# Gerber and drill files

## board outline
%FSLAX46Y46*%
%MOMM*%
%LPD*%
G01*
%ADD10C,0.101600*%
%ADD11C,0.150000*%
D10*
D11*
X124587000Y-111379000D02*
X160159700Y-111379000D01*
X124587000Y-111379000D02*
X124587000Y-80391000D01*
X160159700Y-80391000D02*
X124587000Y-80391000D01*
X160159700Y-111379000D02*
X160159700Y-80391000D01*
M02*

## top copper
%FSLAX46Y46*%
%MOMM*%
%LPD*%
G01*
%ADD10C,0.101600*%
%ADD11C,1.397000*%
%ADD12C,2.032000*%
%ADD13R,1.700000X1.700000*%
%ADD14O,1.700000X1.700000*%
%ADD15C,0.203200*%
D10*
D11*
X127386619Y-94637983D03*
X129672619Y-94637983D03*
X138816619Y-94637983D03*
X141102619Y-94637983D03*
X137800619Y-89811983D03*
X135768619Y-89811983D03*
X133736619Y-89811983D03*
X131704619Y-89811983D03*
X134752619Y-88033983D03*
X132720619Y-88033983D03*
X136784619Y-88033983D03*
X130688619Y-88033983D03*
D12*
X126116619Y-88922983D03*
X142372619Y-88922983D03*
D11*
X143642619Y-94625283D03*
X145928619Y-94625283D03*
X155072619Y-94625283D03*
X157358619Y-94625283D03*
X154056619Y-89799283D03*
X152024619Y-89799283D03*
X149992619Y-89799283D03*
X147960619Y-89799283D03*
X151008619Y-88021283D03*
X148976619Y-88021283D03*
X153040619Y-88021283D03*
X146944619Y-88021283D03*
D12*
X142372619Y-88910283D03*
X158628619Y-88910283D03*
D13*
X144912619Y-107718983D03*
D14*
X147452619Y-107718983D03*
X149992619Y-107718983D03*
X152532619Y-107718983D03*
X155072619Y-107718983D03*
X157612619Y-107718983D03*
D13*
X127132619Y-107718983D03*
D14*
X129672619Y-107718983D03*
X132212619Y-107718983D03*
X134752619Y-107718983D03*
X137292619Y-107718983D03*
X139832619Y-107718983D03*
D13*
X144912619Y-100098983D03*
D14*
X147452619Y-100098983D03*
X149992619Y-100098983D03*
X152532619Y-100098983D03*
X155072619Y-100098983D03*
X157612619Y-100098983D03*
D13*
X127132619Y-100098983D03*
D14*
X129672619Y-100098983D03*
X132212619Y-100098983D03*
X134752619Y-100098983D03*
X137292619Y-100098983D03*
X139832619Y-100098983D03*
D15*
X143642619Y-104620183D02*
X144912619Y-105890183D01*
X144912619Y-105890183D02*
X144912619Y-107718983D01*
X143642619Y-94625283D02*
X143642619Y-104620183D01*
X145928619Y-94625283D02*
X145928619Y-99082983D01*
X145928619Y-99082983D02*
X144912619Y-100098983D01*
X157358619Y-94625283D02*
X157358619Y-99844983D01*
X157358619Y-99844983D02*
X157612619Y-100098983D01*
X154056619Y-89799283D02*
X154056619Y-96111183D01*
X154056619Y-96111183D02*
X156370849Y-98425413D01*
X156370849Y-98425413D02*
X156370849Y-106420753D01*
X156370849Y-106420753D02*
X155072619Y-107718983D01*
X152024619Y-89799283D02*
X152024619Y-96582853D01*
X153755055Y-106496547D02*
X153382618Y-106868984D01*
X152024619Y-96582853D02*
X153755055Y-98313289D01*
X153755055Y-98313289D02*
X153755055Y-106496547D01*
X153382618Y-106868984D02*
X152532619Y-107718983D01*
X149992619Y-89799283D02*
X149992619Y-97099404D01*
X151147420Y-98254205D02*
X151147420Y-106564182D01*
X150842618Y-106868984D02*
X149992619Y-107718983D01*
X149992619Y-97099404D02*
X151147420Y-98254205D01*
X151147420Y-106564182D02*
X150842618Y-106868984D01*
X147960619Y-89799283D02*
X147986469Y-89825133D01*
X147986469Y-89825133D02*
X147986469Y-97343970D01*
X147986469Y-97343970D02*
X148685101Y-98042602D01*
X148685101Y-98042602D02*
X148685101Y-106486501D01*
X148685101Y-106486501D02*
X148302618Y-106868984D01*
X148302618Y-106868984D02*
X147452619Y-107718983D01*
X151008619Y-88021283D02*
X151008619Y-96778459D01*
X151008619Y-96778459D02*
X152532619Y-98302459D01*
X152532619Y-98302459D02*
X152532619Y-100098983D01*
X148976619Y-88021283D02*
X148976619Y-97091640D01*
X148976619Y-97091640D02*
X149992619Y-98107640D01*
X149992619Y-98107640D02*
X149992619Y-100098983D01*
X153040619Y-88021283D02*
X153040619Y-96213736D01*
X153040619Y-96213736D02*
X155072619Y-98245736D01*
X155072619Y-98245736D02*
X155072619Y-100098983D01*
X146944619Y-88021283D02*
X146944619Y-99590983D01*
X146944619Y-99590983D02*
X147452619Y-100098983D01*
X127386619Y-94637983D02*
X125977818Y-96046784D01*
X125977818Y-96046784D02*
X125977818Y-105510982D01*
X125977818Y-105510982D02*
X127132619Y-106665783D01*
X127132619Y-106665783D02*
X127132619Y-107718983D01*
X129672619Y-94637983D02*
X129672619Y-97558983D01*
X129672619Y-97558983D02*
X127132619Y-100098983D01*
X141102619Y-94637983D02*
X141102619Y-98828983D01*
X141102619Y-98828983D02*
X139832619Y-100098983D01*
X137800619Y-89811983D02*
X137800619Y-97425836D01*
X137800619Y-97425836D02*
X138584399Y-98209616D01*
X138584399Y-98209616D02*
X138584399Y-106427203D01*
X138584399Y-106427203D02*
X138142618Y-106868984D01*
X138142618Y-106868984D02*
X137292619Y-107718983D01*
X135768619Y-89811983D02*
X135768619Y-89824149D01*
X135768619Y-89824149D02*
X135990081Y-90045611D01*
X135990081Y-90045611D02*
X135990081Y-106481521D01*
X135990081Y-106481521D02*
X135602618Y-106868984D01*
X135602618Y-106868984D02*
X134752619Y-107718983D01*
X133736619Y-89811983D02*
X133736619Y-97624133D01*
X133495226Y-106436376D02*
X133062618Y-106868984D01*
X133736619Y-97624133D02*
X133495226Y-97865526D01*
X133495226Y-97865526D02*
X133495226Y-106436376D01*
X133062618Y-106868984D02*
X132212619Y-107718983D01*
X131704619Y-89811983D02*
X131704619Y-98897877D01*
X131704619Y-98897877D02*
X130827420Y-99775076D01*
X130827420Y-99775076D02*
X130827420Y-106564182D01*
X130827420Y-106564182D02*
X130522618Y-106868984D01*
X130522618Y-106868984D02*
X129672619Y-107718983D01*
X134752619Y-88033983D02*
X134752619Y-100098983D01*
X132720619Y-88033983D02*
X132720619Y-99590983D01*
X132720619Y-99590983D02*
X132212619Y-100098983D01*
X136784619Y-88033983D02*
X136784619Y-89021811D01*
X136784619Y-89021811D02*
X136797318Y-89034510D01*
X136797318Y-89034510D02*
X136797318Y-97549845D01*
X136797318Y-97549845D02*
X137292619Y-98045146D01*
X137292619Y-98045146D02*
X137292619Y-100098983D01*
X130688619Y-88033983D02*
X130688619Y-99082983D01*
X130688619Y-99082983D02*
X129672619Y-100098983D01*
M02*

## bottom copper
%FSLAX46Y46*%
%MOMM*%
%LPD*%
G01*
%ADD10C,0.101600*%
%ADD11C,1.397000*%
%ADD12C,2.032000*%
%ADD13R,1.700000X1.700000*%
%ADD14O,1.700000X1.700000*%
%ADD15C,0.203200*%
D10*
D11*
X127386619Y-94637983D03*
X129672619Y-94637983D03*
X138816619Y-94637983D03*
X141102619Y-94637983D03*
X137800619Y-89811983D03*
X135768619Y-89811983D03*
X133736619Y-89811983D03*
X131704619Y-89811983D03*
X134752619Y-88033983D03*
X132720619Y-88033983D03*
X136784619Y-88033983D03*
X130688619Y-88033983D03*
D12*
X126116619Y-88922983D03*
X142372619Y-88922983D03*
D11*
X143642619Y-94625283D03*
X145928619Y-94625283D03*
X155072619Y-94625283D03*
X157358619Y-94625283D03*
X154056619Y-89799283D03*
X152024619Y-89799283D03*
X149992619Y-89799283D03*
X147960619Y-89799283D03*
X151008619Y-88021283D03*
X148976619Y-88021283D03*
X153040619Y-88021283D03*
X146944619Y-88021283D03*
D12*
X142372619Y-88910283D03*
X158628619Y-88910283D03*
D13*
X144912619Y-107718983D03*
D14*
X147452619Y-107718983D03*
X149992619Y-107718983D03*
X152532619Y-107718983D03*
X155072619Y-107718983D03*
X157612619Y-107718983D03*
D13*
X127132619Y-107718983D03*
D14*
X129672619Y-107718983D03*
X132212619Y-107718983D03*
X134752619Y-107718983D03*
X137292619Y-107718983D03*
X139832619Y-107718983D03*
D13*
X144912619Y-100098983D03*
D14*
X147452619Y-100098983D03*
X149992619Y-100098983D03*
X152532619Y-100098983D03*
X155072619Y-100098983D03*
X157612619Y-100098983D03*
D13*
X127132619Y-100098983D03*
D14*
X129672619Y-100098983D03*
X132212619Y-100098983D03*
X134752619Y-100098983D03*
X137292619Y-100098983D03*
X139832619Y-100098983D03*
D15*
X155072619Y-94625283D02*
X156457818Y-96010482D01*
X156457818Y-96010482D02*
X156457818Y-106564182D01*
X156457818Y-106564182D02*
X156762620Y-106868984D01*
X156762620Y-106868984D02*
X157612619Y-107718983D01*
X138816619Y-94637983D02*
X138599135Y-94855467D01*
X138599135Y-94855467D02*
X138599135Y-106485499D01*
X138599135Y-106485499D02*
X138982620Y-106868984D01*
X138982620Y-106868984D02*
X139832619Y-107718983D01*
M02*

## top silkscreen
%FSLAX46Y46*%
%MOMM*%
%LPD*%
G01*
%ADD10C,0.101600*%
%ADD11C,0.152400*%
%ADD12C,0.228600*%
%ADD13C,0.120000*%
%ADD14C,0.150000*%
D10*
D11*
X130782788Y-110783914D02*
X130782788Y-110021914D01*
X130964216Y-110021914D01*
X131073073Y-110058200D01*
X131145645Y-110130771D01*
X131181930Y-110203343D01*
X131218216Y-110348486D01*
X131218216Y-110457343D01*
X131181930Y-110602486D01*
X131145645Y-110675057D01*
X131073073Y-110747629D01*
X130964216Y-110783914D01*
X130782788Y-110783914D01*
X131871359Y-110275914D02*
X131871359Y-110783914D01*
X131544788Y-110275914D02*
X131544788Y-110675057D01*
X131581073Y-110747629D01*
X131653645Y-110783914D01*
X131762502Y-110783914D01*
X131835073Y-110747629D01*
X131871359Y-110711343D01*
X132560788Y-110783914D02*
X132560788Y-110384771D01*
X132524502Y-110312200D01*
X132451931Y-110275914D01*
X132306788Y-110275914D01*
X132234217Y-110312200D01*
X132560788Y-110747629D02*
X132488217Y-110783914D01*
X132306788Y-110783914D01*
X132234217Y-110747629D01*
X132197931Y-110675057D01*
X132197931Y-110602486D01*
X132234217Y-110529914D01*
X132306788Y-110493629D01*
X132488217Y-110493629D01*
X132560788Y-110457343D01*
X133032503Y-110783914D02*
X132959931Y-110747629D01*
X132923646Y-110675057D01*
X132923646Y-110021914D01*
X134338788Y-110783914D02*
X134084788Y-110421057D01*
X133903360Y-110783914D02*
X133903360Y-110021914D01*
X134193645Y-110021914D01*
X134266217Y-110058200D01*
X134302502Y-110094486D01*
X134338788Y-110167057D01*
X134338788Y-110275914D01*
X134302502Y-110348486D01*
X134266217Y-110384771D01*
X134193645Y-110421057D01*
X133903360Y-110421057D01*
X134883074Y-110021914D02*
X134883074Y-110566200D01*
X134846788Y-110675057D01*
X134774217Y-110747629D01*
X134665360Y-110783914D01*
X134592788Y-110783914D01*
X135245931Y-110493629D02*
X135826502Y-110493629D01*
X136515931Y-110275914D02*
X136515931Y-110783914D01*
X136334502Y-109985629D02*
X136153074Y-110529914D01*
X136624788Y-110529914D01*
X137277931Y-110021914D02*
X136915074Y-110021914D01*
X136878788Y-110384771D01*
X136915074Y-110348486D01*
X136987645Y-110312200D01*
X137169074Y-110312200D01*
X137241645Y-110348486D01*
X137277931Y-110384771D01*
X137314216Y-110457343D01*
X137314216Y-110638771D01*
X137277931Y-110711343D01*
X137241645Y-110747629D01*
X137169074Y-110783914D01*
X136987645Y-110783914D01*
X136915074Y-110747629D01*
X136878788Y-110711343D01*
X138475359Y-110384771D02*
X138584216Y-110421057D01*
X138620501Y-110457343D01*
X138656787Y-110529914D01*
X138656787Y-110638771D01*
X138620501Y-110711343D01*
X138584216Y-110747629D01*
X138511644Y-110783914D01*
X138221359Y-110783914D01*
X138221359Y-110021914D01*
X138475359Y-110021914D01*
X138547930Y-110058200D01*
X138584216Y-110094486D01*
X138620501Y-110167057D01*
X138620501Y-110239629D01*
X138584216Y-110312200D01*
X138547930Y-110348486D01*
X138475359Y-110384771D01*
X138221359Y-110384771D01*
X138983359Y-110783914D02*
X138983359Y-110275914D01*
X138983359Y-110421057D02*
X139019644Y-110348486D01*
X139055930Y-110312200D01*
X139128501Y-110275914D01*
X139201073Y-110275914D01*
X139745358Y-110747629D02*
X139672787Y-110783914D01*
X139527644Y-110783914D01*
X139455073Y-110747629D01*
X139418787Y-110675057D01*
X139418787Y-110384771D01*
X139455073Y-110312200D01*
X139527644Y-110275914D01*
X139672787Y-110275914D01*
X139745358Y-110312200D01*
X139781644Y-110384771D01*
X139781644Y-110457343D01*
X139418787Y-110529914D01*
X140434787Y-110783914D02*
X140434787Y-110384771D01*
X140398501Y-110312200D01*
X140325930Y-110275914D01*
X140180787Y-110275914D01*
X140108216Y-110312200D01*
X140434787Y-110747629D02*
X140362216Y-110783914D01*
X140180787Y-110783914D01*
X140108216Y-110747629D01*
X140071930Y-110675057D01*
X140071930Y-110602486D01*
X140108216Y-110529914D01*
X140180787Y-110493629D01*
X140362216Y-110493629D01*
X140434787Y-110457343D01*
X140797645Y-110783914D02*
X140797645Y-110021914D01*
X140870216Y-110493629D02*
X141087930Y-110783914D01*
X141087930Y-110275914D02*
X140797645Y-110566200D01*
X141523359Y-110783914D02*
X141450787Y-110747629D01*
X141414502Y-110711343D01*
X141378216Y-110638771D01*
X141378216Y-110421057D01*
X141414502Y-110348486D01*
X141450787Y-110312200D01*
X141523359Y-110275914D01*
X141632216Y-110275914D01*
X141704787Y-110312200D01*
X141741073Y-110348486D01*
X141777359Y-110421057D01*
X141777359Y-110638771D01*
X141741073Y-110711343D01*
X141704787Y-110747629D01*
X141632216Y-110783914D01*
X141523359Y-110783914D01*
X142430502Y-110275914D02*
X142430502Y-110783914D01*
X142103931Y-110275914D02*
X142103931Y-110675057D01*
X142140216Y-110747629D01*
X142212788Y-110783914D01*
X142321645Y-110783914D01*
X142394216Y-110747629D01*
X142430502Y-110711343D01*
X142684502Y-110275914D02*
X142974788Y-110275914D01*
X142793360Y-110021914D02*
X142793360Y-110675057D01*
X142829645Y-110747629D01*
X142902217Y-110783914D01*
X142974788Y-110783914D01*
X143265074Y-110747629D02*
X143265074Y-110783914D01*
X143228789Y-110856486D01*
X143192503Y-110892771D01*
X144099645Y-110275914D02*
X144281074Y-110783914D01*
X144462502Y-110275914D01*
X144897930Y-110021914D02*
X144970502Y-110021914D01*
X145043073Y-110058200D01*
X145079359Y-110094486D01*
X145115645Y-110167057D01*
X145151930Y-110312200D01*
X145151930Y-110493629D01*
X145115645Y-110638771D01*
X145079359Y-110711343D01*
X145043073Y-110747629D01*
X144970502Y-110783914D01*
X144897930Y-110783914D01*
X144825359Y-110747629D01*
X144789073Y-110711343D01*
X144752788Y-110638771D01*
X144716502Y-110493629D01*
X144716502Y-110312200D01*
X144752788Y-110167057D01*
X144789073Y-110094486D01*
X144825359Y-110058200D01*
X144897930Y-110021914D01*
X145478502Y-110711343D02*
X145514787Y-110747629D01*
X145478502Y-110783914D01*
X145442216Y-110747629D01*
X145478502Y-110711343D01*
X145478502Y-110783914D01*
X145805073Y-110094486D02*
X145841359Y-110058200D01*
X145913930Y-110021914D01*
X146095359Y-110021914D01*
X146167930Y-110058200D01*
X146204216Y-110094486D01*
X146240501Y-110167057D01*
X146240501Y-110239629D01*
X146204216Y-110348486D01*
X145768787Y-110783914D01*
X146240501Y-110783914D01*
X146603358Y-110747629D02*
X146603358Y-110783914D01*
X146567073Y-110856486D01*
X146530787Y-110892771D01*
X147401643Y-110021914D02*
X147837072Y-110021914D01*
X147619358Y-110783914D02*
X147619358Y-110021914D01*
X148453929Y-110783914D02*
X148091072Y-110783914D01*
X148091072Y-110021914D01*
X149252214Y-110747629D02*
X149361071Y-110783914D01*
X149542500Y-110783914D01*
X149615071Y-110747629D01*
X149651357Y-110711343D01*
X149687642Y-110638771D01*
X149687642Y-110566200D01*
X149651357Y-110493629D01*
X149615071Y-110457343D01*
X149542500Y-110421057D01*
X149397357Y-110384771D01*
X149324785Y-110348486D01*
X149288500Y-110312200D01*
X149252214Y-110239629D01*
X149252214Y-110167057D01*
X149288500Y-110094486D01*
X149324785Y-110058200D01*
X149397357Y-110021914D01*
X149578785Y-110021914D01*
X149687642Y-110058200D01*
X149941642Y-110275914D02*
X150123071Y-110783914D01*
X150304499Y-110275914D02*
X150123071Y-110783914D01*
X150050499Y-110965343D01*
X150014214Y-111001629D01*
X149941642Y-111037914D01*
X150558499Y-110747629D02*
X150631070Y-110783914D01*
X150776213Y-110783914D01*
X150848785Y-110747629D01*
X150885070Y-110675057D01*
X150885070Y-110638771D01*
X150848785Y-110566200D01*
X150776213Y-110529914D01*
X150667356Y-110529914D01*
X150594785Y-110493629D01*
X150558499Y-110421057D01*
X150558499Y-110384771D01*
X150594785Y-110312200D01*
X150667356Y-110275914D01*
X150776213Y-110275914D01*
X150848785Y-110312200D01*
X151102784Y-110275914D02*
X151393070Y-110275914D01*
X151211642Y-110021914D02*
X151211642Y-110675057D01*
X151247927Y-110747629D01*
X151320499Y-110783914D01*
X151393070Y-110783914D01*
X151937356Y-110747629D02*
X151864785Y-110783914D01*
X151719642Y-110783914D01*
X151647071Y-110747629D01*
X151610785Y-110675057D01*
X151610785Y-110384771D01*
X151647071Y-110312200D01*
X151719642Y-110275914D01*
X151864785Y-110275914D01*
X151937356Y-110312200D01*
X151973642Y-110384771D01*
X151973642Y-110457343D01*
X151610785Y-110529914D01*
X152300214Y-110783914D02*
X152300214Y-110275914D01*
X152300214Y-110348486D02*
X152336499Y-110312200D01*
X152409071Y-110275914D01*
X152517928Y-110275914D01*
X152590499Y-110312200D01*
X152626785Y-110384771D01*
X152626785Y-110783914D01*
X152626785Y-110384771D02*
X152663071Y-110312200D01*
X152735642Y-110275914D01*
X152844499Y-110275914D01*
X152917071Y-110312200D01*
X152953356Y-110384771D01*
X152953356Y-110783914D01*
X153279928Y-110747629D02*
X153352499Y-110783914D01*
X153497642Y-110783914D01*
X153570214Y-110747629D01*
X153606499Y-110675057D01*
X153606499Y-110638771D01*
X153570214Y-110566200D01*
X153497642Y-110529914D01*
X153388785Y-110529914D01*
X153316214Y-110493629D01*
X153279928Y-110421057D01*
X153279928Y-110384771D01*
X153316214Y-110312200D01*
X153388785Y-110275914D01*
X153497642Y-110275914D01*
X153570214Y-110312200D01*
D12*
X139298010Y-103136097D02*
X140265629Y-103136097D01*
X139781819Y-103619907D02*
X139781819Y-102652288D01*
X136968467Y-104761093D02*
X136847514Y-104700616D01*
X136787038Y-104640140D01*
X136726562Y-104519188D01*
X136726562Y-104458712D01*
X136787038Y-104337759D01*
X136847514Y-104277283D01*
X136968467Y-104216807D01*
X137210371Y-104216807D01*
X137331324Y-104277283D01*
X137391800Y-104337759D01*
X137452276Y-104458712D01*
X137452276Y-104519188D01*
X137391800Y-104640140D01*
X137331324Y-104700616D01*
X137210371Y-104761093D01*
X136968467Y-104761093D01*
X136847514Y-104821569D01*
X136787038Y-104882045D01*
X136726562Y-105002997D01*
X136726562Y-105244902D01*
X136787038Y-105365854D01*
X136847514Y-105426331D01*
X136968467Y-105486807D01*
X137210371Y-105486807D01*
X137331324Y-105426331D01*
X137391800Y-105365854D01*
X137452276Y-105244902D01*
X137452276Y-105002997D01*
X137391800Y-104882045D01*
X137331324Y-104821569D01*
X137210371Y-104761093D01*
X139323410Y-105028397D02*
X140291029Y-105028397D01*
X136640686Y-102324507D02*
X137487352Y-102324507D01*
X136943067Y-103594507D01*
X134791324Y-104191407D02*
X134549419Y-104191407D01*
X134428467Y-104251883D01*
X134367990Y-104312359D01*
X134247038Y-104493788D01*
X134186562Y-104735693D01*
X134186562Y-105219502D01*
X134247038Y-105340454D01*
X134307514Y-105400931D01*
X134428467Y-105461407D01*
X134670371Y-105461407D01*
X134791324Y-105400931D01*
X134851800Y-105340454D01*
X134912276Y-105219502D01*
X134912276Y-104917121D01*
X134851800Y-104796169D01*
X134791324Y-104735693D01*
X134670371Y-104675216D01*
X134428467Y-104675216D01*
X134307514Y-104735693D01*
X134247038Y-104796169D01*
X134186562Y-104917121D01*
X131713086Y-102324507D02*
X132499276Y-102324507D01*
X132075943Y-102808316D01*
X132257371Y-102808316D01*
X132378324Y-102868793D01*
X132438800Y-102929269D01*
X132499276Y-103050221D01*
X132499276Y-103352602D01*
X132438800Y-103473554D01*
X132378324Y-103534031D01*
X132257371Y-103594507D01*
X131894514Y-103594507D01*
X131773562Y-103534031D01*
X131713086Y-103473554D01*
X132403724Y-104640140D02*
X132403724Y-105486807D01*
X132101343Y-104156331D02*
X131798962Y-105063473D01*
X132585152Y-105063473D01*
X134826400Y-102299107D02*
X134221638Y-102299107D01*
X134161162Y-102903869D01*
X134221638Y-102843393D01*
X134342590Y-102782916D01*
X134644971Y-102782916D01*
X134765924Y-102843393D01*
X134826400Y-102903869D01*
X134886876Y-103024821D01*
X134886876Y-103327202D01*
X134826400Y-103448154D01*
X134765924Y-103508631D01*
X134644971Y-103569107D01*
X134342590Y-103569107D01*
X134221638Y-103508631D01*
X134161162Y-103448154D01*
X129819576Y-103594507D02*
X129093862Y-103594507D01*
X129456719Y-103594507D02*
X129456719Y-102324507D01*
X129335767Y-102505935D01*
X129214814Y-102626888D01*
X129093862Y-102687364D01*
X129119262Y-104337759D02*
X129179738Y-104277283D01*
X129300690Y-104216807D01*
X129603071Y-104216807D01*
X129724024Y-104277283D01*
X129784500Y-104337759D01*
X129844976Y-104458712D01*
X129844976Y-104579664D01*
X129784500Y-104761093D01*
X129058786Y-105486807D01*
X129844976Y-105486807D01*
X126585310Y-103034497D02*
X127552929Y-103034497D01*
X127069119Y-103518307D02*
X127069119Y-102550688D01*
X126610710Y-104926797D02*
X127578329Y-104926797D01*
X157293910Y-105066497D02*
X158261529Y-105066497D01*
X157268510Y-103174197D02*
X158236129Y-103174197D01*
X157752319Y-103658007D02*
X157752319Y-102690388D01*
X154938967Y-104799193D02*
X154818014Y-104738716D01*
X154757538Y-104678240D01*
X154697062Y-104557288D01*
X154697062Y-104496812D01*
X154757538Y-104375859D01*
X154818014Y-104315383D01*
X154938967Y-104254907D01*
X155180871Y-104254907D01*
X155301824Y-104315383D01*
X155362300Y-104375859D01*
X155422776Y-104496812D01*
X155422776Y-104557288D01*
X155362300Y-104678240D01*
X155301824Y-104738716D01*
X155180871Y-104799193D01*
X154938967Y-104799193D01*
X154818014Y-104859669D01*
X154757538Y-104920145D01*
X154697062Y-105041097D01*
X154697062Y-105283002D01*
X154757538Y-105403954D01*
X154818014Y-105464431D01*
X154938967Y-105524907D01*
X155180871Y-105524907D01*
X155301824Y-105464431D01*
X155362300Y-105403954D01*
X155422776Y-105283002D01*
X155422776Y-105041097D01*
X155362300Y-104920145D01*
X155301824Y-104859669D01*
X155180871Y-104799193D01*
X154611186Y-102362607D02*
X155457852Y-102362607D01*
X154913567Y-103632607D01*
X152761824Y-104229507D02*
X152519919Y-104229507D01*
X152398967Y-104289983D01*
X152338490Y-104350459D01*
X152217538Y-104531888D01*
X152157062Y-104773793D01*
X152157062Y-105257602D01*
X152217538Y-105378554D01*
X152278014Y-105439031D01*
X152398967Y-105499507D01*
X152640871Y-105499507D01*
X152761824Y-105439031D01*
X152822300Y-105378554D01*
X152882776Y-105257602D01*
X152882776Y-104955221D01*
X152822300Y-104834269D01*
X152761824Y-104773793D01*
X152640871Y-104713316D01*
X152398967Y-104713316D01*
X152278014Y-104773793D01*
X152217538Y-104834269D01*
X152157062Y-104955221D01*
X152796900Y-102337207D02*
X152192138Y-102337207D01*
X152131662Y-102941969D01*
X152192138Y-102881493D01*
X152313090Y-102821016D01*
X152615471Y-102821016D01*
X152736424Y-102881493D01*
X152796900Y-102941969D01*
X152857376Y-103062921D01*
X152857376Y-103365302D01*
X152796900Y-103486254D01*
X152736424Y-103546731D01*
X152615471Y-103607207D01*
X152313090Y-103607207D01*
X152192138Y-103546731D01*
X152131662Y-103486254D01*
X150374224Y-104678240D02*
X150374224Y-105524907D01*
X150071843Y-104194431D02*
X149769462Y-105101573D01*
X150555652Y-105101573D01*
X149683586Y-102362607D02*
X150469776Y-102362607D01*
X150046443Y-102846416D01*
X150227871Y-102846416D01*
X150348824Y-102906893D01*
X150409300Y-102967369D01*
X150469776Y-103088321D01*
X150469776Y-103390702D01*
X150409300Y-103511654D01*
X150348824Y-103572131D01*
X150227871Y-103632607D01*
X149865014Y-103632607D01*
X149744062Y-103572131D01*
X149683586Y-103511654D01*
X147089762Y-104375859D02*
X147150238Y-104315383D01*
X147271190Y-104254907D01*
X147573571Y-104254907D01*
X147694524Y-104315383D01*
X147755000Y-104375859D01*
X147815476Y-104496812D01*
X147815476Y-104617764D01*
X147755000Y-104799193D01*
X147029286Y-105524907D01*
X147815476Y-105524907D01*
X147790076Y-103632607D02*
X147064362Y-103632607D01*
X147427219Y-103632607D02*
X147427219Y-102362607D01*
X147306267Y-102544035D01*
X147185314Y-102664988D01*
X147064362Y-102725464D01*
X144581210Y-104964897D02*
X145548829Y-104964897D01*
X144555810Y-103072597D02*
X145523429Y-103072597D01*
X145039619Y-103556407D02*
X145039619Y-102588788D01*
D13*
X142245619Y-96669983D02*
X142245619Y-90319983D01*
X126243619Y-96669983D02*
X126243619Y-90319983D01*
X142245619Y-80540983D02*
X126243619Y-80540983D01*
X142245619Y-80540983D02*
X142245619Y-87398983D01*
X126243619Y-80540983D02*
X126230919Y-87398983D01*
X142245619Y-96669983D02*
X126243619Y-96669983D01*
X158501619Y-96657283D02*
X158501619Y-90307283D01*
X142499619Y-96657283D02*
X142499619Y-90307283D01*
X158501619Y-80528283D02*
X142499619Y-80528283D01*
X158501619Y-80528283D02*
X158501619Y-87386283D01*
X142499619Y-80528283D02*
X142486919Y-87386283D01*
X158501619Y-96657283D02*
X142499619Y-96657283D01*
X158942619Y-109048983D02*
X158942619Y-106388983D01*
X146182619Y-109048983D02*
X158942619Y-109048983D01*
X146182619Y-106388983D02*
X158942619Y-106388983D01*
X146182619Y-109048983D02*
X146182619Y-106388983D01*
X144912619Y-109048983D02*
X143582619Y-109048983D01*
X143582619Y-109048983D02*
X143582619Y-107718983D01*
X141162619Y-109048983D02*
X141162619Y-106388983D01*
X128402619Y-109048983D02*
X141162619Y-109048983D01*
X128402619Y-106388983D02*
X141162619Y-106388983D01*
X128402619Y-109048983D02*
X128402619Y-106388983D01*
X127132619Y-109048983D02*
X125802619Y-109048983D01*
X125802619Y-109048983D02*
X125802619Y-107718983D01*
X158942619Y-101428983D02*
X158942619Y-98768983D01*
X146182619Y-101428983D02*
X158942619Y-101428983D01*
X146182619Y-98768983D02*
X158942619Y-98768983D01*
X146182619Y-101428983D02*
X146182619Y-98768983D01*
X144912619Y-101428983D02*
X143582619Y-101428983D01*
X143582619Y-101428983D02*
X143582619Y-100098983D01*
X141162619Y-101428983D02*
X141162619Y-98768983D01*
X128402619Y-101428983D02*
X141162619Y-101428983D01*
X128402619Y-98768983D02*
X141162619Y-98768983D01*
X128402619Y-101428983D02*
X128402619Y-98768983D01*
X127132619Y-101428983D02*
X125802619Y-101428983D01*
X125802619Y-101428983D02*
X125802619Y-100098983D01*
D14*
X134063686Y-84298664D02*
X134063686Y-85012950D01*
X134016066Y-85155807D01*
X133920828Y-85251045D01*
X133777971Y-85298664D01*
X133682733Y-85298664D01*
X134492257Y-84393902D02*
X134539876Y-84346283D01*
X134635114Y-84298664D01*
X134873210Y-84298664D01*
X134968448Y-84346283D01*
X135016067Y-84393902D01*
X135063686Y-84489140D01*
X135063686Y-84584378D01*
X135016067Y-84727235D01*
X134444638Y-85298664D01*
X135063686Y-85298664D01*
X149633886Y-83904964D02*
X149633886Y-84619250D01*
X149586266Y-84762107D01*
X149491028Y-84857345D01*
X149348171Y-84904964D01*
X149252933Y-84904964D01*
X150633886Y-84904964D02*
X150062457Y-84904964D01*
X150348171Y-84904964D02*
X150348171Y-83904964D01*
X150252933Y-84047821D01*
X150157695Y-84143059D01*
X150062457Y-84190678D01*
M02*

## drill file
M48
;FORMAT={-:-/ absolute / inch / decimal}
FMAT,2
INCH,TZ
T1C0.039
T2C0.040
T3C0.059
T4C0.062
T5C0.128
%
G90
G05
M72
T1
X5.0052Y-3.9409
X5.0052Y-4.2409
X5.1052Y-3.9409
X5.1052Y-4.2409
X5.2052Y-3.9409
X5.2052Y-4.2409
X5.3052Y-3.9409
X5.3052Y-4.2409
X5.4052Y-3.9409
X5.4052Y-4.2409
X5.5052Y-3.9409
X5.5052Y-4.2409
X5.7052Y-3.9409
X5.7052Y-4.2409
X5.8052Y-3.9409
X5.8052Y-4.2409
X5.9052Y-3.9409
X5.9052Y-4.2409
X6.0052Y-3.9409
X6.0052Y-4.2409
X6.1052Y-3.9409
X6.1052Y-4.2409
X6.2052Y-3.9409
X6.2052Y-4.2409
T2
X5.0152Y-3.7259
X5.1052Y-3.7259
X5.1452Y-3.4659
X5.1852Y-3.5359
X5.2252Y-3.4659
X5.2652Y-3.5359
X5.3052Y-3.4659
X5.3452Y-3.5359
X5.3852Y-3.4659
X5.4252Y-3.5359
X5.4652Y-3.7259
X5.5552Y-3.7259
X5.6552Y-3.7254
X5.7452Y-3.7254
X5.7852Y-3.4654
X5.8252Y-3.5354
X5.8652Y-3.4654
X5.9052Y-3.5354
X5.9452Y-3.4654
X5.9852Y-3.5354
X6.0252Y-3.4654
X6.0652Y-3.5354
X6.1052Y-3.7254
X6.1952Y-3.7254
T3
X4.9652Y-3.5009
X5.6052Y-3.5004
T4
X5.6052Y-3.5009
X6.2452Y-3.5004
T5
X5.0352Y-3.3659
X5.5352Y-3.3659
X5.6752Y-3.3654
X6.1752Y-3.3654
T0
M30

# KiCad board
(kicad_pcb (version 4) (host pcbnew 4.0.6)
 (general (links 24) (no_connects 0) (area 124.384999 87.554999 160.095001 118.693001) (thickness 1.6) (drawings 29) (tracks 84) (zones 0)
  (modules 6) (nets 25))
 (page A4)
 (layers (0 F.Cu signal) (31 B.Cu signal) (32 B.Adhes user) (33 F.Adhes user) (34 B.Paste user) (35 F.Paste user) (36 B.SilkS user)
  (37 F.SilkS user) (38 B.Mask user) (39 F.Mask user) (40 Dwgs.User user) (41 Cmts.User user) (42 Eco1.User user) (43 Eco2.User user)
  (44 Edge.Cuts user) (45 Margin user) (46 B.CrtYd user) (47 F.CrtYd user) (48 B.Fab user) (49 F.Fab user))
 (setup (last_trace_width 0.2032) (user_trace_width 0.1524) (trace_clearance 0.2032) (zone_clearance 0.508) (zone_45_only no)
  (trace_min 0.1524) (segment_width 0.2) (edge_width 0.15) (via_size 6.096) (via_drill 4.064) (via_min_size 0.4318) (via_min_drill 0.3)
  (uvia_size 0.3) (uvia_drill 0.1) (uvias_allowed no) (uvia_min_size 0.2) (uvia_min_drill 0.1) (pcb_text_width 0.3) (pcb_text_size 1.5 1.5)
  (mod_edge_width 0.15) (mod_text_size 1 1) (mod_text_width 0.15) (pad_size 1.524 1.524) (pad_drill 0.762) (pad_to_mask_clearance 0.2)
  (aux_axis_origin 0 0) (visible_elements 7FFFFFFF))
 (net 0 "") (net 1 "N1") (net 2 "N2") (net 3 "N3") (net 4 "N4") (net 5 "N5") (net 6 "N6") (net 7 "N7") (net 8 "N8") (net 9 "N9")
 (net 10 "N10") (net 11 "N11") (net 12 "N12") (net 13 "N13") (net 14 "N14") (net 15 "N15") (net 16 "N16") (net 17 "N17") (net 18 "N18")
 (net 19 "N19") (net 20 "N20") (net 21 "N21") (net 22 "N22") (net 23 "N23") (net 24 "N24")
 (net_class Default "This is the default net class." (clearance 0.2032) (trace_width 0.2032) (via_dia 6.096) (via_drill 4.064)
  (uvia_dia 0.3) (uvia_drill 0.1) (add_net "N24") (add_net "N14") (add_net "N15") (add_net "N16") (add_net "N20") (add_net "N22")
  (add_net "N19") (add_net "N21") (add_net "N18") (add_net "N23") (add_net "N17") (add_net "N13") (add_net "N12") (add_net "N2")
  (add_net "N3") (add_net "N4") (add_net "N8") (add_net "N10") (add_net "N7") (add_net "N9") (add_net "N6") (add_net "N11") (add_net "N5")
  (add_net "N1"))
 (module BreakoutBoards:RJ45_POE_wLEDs (layer F.Cu) (at 140.594619 85.493983 180)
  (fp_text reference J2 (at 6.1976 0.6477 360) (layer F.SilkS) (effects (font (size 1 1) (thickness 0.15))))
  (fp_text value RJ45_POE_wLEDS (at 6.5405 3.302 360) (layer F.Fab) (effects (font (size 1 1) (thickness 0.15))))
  (fp_line (start -1.651 -11.176) (end -1.651 -4.826) (layer F.SilkS) (width 0.12))
  (fp_line (start 14.351 -11.176) (end 14.351 -4.826) (layer F.SilkS) (width 0.12))
  (fp_line (start -1.651 4.953) (end 14.351 4.953) (layer F.SilkS) (width 0.12))
  (fp_line (start -1.651 4.953) (end -1.651 -1.905) (layer F.SilkS) (width 0.12))
  (fp_line (start 14.351 4.953) (end 14.3637 -1.905) (layer F.SilkS) (width 0.12))
  (fp_line (start -1.651 -11.176) (end 14.351 -11.176) (layer F.SilkS) (width 0.12))
  (pad 9 thru_hole circle (at 13.208 -9.144) (size 1.397 1.397) (drill 1.016) (layers *.Cu *.Mask) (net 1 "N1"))
  (pad 10 thru_hole circle (at 10.922 -9.144) (size 1.397 1.397) (drill 1.016) (layers *.Cu *.Mask) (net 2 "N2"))
  (pad 11 thru_hole circle (at 1.778 -9.144) (size 1.397 1.397) (drill 1.016) (layers *.Cu *.Mask) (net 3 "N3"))
  (pad 12 thru_hole circle (at -0.508 -9.144) (size 1.397 1.397) (drill 1.016) (layers *.Cu *.Mask) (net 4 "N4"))
  (pad 8 thru_hole circle (at 2.794 -4.318) (size 1.397 1.397) (drill 1.016) (layers *.Cu *.Mask) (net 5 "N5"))
  (pad 6 thru_hole circle (at 4.826 -4.318) (size 1.397 1.397) (drill 1.016) (layers *.Cu *.Mask) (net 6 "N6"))
  (pad 4 thru_hole circle (at 6.858 -4.318) (size 1.397 1.397) (drill 1.016) (layers *.Cu *.Mask) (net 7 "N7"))
  (pad 2 thru_hole circle (at 8.89 -4.318) (size 1.397 1.397) (drill 1.016) (layers *.Cu *.Mask) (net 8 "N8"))
  (pad 5 thru_hole circle (at 5.842 -2.54) (size 1.397 1.397) (drill 1.016) (layers *.Cu *.Mask) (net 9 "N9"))
  (pad 3 thru_hole circle (at 7.874 -2.54) (size 1.397 1.397) (drill 1.016) (layers *.Cu *.Mask) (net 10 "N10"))
  (pad 7 thru_hole circle (at 3.81 -2.54) (size 1.397 1.397) (drill 1.016) (layers *.Cu *.Mask) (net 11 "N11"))
  (pad 1 thru_hole circle (at 9.906 -2.54) (size 1.397 1.397) (drill 1.016) (layers *.Cu *.Mask) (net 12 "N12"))
  (pad "" np_thru_hole circle (at 12.7 0) (size 3.2512 3.2512) (drill 3.2512) (layers *.Cu *.Mask))
  (pad "" np_thru_hole circle (at 0 0) (size 3.2512 3.2512) (drill 3.2512) (layers *.Cu *.Mask))
  (pad 13 thru_hole circle (at 14.478 -3.429) (size 2.032 2.032) (drill 1.5) (layers *.Cu *.Mask))
  (pad 14 thru_hole circle (at -1.778 -3.429) (size 2.032 2.032) (drill 1.5748) (layers *.Cu *.Mask)))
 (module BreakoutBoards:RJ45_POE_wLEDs (layer F.Cu) (at 156.850619 85.481283 180)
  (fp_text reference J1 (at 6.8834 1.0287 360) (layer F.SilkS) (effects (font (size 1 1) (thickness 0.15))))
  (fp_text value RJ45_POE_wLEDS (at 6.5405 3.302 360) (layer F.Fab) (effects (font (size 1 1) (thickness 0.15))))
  (fp_line (start -1.651 -11.176) (end -1.651 -4.826) (layer F.SilkS) (width 0.12))
  (fp_line (start 14.351 -11.176) (end 14.351 -4.826) (layer F.SilkS) (width 0.12))
  (fp_line (start -1.651 4.953) (end 14.351 4.953) (layer F.SilkS) (width 0.12))
  (fp_line (start -1.651 4.953) (end -1.651 -1.905) (layer F.SilkS) (width 0.12))
  (fp_line (start 14.351 4.953) (end 14.3637 -1.905) (layer F.SilkS) (width 0.12))
  (fp_line (start -1.651 -11.176) (end 14.351 -11.176) (layer F.SilkS) (width 0.12))
  (pad 9 thru_hole circle (at 13.208 -9.144) (size 1.397 1.397) (drill 1.016) (layers *.Cu *.Mask) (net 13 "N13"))
  (pad 10 thru_hole circle (at 10.922 -9.144) (size 1.397 1.397) (drill 1.016) (layers *.Cu *.Mask) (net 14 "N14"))
  (pad 11 thru_hole circle (at 1.778 -9.144) (size 1.397 1.397) (drill 1.016) (layers *.Cu *.Mask) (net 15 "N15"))
  (pad 12 thru_hole circle (at -0.508 -9.144) (size 1.397 1.397) (drill 1.016) (layers *.Cu *.Mask) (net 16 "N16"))
  (pad 8 thru_hole circle (at 2.794 -4.318) (size 1.397 1.397) (drill 1.016) (layers *.Cu *.Mask) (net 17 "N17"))
  (pad 6 thru_hole circle (at 4.826 -4.318) (size 1.397 1.397) (drill 1.016) (layers *.Cu *.Mask) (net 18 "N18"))
  (pad 4 thru_hole circle (at 6.858 -4.318) (size 1.397 1.397) (drill 1.016) (layers *.Cu *.Mask) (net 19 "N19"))
  (pad 2 thru_hole circle (at 8.89 -4.318) (size 1.397 1.397) (drill 1.016) (layers *.Cu *.Mask) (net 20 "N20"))
  (pad 5 thru_hole circle (at 5.842 -2.54) (size 1.397 1.397) (drill 1.016) (layers *.Cu *.Mask) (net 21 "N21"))
  (pad 3 thru_hole circle (at 7.874 -2.54) (size 1.397 1.397) (drill 1.016) (layers *.Cu *.Mask) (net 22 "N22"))
  (pad 7 thru_hole circle (at 3.81 -2.54) (size 1.397 1.397) (drill 1.016) (layers *.Cu *.Mask) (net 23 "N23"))
  (pad 1 thru_hole circle (at 9.906 -2.54) (size 1.397 1.397) (drill 1.016) (layers *.Cu *.Mask) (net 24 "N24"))
  (pad "" np_thru_hole circle (at 12.7 0) (size 3.2512 3.2512) (drill 3.2512) (layers *.Cu *.Mask))
  (pad "" np_thru_hole circle (at 0 0) (size 3.2512 3.2512) (drill 3.2512) (layers *.Cu *.Mask))
  (pad 13 thru_hole circle (at 14.478 -3.429) (size 2.032 2.032) (drill 1.5) (layers *.Cu *.Mask))
  (pad 14 thru_hole circle (at -1.778 -3.429) (size 2.032 2.032) (drill 1.5748) (layers *.Cu *.Mask)))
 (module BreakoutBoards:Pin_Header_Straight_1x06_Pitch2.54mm (layer F.Cu) (at 144.912619 107.718983 90)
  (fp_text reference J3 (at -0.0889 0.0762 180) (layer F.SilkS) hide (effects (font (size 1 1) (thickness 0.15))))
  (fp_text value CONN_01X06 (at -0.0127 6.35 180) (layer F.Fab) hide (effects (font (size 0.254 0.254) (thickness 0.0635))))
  (fp_line (start -1.33 14.03) (end 1.33 14.03) (layer F.SilkS) (width 0.12))
  (fp_line (start -1.33 1.27) (end -1.33 14.03) (layer F.SilkS) (width 0.12))
  (fp_line (start 1.33 1.27) (end 1.33 14.03) (layer F.SilkS) (width 0.12))
  (fp_line (start -1.33 1.27) (end 1.33 1.27) (layer F.SilkS) (width 0.12))
  (fp_line (start -1.33 0) (end -1.33 -1.33) (layer F.SilkS) (width 0.12))
  (fp_line (start -1.33 -1.33) (end 0 -1.33) (layer F.SilkS) (width 0.12))
  (pad 1 thru_hole rect (at 0 0 90) (size 1.7 1.7) (drill 1) (layers *.Cu *.Mask) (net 13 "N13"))
  (pad 2 thru_hole oval (at 0 2.54 90) (size 1.7 1.7) (drill 1) (layers *.Cu *.Mask) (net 20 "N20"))
  (pad 3 thru_hole oval (at 0 5.08 90) (size 1.7 1.7) (drill 1) (layers *.Cu *.Mask) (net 19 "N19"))
  (pad 4 thru_hole oval (at 0 7.62 90) (size 1.7 1.7) (drill 1) (layers *.Cu *.Mask) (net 18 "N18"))
  (pad 5 thru_hole oval (at 0 10.16 90) (size 1.7 1.7) (drill 1) (layers *.Cu *.Mask) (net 17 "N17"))
  (pad 6 thru_hole oval (at 0 12.7 90) (size 1.7 1.7) (drill 1) (layers *.Cu *.Mask) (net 15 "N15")))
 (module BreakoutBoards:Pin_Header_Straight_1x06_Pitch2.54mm (layer F.Cu) (at 127.132619 107.718983 90)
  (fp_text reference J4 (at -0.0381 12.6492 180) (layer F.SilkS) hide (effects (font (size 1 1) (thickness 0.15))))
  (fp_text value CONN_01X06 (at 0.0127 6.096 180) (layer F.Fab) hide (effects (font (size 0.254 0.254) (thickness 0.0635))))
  (fp_line (start -1.33 14.03) (end 1.33 14.03) (layer F.SilkS) (width 0.12))
  (fp_line (start -1.33 1.27) (end -1.33 14.03) (layer F.SilkS) (width 0.12))
  (fp_line (start 1.33 1.27) (end 1.33 14.03) (layer F.SilkS) (width 0.12))
  (fp_line (start -1.33 1.27) (end 1.33 1.27) (layer F.SilkS) (width 0.12))
  (fp_line (start -1.33 0) (end -1.33 -1.33) (layer F.SilkS) (width 0.12))
  (fp_line (start -1.33 -1.33) (end 0 -1.33) (layer F.SilkS) (width 0.12))
  (pad 1 thru_hole rect (at 0 0 90) (size 1.7 1.7) (drill 1) (layers *.Cu *.Mask) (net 1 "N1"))
  (pad 2 thru_hole oval (at 0 2.54 90) (size 1.7 1.7) (drill 1) (layers *.Cu *.Mask) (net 8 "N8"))
  (pad 3 thru_hole oval (at 0 5.08 90) (size 1.7 1.7) (drill 1) (layers *.Cu *.Mask) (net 7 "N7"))
  (pad 4 thru_hole oval (at 0 7.62 90) (size 1.7 1.7) (drill 1) (layers *.Cu *.Mask) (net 6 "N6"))
  (pad 5 thru_hole oval (at 0 10.16 90) (size 1.7 1.7) (drill 1) (layers *.Cu *.Mask) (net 5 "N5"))
  (pad 6 thru_hole oval (at 0 12.7 90) (size 1.7 1.7) (drill 1) (layers *.Cu *.Mask) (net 3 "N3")))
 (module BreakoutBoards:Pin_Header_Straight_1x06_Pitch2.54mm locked (layer F.Cu) (at 144.912619 100.098983 90)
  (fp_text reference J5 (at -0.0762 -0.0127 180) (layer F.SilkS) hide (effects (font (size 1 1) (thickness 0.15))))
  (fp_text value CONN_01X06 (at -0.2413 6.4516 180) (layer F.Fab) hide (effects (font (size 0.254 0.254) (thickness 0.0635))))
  (fp_line (start -1.33 14.03) (end 1.33 14.03) (layer F.SilkS) (width 0.12))
  (fp_line (start -1.33 1.27) (end -1.33 14.03) (layer F.SilkS) (width 0.12))
  (fp_line (start 1.33 1.27) (end 1.33 14.03) (layer F.SilkS) (width 0.12))
  (fp_line (start -1.33 1.27) (end 1.33 1.27) (layer F.SilkS) (width 0.12))
  (fp_line (start -1.33 0) (end -1.33 -1.33) (layer F.SilkS) (width 0.12))
  (fp_line (start -1.33 -1.33) (end 0 -1.33) (layer F.SilkS) (width 0.12))
  (pad 1 thru_hole rect (at 0 0 90) (size 1.7 1.7) (drill 1) (layers *.Cu *.Mask) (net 14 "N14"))
  (pad 2 thru_hole oval (at 0 2.54 90) (size 1.7 1.7) (drill 1) (layers *.Cu *.Mask) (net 24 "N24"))
  (pad 3 thru_hole oval (at 0 5.08 90) (size 1.7 1.7) (drill 1) (layers *.Cu *.Mask) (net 22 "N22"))
  (pad 4 thru_hole oval (at 0 7.62 90) (size 1.7 1.7) (drill 1) (layers *.Cu *.Mask) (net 21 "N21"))
  (pad 5 thru_hole oval (at 0 10.16 90) (size 1.7 1.7) (drill 1) (layers *.Cu *.Mask) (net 23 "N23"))
  (pad 6 thru_hole oval (at 0 12.7 90) (size 1.7 1.7) (drill 1) (layers *.Cu *.Mask) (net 16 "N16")))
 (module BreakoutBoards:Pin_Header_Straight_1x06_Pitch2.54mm (layer F.Cu) (at 127.132619 100.098983 90)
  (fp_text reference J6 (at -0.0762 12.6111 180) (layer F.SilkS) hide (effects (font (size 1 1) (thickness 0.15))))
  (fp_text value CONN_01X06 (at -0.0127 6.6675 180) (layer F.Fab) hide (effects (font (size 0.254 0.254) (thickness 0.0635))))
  (fp_line (start -1.33 14.03) (end 1.33 14.03) (layer F.SilkS) (width 0.12))
  (fp_line (start -1.33 1.27) (end -1.33 14.03) (layer F.SilkS) (width 0.12))
  (fp_line (start 1.33 1.27) (end 1.33 14.03) (layer F.SilkS) (width 0.12))
  (fp_line (start -1.33 1.27) (end 1.33 1.27) (layer F.SilkS) (width 0.12))
  (fp_line (start -1.33 0) (end -1.33 -1.33) (layer F.SilkS) (width 0.12))
  (fp_line (start -1.33 -1.33) (end 0 -1.33) (layer F.SilkS) (width 0.12))
  (pad 1 thru_hole rect (at 0 0 90) (size 1.7 1.7) (drill 1) (layers *.Cu *.Mask) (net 2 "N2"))
  (pad 2 thru_hole oval (at 0 2.54 90) (size 1.7 1.7) (drill 1) (layers *.Cu *.Mask) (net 12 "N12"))
  (pad 3 thru_hole oval (at 0 5.08 90) (size 1.7 1.7) (drill 1) (layers *.Cu *.Mask) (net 10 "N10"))
  (pad 4 thru_hole oval (at 0 7.62 90) (size 1.7 1.7) (drill 1) (layers *.Cu *.Mask) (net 9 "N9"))
  (pad 5 thru_hole oval (at 0 10.16 90) (size 1.7 1.7) (drill 1) (layers *.Cu *.Mask) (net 11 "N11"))
  (pad 6 thru_hole oval (at 0 12.7 90) (size 1.7 1.7) (drill 1) (layers *.Cu *.Mask) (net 4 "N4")))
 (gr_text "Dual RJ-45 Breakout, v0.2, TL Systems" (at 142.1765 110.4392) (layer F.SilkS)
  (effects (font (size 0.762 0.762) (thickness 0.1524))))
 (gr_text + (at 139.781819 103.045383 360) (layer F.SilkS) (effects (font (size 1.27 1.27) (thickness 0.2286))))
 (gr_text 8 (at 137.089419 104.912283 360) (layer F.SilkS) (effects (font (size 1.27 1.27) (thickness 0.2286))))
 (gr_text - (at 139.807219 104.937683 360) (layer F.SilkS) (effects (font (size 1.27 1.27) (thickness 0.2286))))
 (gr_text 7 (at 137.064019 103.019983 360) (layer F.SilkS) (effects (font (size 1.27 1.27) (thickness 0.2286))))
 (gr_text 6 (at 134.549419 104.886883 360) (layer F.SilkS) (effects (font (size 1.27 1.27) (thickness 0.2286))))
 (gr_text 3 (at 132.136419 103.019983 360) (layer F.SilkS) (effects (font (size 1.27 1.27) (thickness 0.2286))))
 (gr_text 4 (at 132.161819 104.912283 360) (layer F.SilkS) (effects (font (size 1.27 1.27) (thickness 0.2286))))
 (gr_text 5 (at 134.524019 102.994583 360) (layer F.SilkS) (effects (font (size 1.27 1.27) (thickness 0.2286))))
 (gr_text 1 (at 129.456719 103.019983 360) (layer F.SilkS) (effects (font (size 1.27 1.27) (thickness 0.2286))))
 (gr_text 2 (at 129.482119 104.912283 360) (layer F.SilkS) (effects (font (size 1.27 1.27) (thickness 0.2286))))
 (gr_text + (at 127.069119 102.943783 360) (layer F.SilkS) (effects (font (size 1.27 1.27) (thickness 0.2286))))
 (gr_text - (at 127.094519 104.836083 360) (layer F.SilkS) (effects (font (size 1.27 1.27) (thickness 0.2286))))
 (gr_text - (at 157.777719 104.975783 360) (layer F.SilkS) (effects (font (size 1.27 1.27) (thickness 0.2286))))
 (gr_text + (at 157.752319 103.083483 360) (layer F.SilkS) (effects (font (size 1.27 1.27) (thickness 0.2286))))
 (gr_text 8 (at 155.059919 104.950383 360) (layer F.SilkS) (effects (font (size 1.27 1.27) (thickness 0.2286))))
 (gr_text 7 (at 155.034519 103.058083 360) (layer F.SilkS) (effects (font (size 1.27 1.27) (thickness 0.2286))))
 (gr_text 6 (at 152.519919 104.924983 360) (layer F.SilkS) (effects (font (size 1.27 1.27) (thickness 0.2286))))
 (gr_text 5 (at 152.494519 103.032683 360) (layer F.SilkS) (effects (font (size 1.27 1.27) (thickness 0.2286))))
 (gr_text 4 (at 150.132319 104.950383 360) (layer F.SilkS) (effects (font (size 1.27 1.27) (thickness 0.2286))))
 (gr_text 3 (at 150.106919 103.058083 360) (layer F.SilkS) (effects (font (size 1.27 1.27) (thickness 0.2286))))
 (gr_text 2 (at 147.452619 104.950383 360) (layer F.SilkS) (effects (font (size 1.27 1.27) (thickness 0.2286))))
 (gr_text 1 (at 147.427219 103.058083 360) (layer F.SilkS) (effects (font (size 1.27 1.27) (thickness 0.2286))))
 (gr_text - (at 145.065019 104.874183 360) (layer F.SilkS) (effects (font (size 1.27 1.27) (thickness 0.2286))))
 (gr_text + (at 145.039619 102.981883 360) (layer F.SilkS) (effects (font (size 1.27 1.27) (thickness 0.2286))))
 (gr_line (start 124.587 111.379) (end 160.1597 111.379) (layer Edge.Cuts) (width 0.15))
 (gr_line (start 124.587 111.379) (end 124.587 80.391) (layer Edge.Cuts) (width 0.15))
 (gr_line (start 160.1597 80.391) (end 124.587 80.391) (layer Edge.Cuts) (width 0.15))
 (gr_line (start 160.1597 111.379) (end 160.1597 80.391) (layer Edge.Cuts) (width 0.15))
 (segment (start 143.642619 104.620183) (end 144.912619 105.890183) (width 0.2032) (layer F.Cu) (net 13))
 (segment (start 144.912619 105.890183) (end 144.912619 107.718983) (width 0.2032) (layer F.Cu) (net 13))
 (segment (start 143.642619 94.625283) (end 143.642619 104.620183) (width 0.2032) (layer F.Cu) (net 13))
 (segment (start 145.928619 94.625283) (end 145.928619 99.082983) (width 0.2032) (layer F.Cu) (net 14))
 (segment (start 145.928619 99.082983) (end 144.912619 100.098983) (width 0.2032) (layer F.Cu) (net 14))
 (segment (start 155.072619 94.625283) (end 156.457818 96.010482) (width 0.2032) (layer B.Cu) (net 15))
 (segment (start 156.457818 96.010482) (end 156.457818 106.564182) (width 0.2032) (layer B.Cu) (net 15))
 (segment (start 156.457818 106.564182) (end 156.76262 106.868984) (width 0.2032) (layer B.Cu) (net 15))
 (segment (start 156.76262 106.868984) (end 157.612619 107.718983) (width 0.2032) (layer B.Cu) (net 15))
 (segment (start 157.358619 94.625283) (end 157.358619 99.844983) (width 0.2032) (layer F.Cu) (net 16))
 (segment (start 157.358619 99.844983) (end 157.612619 100.098983) (width 0.2032) (layer F.Cu) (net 16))
 (segment (start 154.056619 89.799283) (end 154.056619 96.111183) (width 0.2032) (layer F.Cu) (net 17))
 (segment (start 154.056619 96.111183) (end 156.370849 98.425413) (width 0.2032) (layer F.Cu) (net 17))
 (segment (start 156.370849 98.425413) (end 156.370849 106.420753) (width 0.2032) (layer F.Cu) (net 17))
 (segment (start 156.370849 106.420753) (end 155.072619 107.718983) (width 0.2032) (layer F.Cu) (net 17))
 (segment (start 152.024619 89.799283) (end 152.024619 96.582853) (width 0.2032) (layer F.Cu) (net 18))
 (segment (start 153.755055 106.496547) (end 153.382618 106.868984) (width 0.2032) (layer F.Cu) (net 18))
 (segment (start 152.024619 96.582853) (end 153.755055 98.313289) (width 0.2032) (layer F.Cu) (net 18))
 (segment (start 153.755055 98.313289) (end 153.755055 106.496547) (width 0.2032) (layer F.Cu) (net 18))
 (segment (start 153.382618 106.868984) (end 152.532619 107.718983) (width 0.2032) (layer F.Cu) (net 18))
 (segment (start 149.992619 89.799283) (end 149.992619 97.099404) (width 0.2032) (layer F.Cu) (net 19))
 (segment (start 151.14742 98.254205) (end 151.14742 106.564182) (width 0.2032) (layer F.Cu) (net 19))
 (segment (start 150.842618 106.868984) (end 149.992619 107.718983) (width 0.2032) (layer F.Cu) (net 19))
 (segment (start 149.992619 97.099404) (end 151.14742 98.254205) (width 0.2032) (layer F.Cu) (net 19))
 (segment (start 151.14742 106.564182) (end 150.842618 106.868984) (width 0.2032) (layer F.Cu) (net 19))
 (segment (start 147.960619 89.799283) (end 147.986469 89.825133) (width 0.2032) (layer F.Cu) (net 20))
 (segment (start 147.986469 89.825133) (end 147.986469 97.34397) (width 0.2032) (layer F.Cu) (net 20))
 (segment (start 147.986469 97.34397) (end 148.685101 98.042602) (width 0.2032) (layer F.Cu) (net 20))
 (segment (start 148.685101 98.042602) (end 148.685101 106.486501) (width 0.2032) (layer F.Cu) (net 20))
 (segment (start 148.685101 106.486501) (end 148.302618 106.868984) (width 0.2032) (layer F.Cu) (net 20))
 (segment (start 148.302618 106.868984) (end 147.452619 107.718983) (width 0.2032) (layer F.Cu) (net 20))
 (segment (start 151.008619 88.021283) (end 151.008619 96.778459) (width 0.2032) (layer F.Cu) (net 21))
 (segment (start 151.008619 96.778459) (end 152.532619 98.302459) (width 0.2032) (layer F.Cu) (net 21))
 (segment (start 152.532619 98.302459) (end 152.532619 100.098983) (width 0.2032) (layer F.Cu) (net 21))
 (segment (start 148.976619 88.021283) (end 148.976619 97.09164) (width 0.2032) (layer F.Cu) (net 22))
 (segment (start 148.976619 97.09164) (end 149.992619 98.10764) (width 0.2032) (layer F.Cu) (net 22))
 (segment (start 149.992619 98.10764) (end 149.992619 100.098983) (width 0.2032) (layer F.Cu) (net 22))
 (segment (start 153.040619 88.021283) (end 153.040619 96.213736) (width 0.2032) (layer F.Cu) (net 23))
 (segment (start 153.040619 96.213736) (end 155.072619 98.245736) (width 0.2032) (layer F.Cu) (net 23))
 (segment (start 155.072619 98.245736) (end 155.072619 100.098983) (width 0.2032) (layer F.Cu) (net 23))
 (segment (start 146.944619 88.021283) (end 146.944619 99.590983) (width 0.2032) (layer F.Cu) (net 24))
 (segment (start 146.944619 99.590983) (end 147.452619 100.098983) (width 0.2032) (layer F.Cu) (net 24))
 (segment (start 127.386619 94.637983) (end 125.977818 96.046784) (width 0.2032) (layer F.Cu) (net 1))
 (segment (start 125.977818 96.046784) (end 125.977818 105.510982) (width 0.2032) (layer F.Cu) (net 1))
 (segment (start 125.977818 105.510982) (end 127.132619 106.665783) (width 0.2032) (layer F.Cu) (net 1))
 (segment (start 127.132619 106.665783) (end 127.132619 107.718983) (width 0.2032) (layer F.Cu) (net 1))
 (segment (start 129.672619 94.637983) (end 129.672619 97.558983) (width 0.2032) (layer F.Cu) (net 2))
 (segment (start 129.672619 97.558983) (end 127.132619 100.098983) (width 0.2032) (layer F.Cu) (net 2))
 (segment (start 138.816619 94.637983) (end 138.599135 94.855467) (width 0.2032) (layer B.Cu) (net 3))
 (segment (start 138.599135 94.855467) (end 138.599135 106.485499) (width 0.2032) (layer B.Cu) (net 3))
 (segment (start 138.599135 106.485499) (end 138.98262 106.868984) (width 0.2032) (layer B.Cu) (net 3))
 (segment (start 138.98262 106.868984) (end 139.832619 107.718983) (width 0.2032) (layer B.Cu) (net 3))
 (segment (start 141.102619 94.637983) (end 141.102619 98.828983) (width 0.2032) (layer F.Cu) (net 4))
 (segment (start 141.102619 98.828983) (end 139.832619 100.098983) (width 0.2032) (layer F.Cu) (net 4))
 (segment (start 137.800619 89.811983) (end 137.800619 97.425836) (width 0.2032) (layer F.Cu) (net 5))
 (segment (start 137.800619 97.425836) (end 138.584399 98.209616) (width 0.2032) (layer F.Cu) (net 5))
 (segment (start 138.584399 98.209616) (end 138.584399 106.427203) (width 0.2032) (layer F.Cu) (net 5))
 (segment (start 138.584399 106.427203) (end 138.142618 106.868984) (width 0.2032) (layer F.Cu) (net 5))
 (segment (start 138.142618 106.868984) (end 137.292619 107.718983) (width 0.2032) (layer F.Cu) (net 5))
 (segment (start 135.768619 89.811983) (end 135.768619 89.824149) (width 0.2032) (layer F.Cu) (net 6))
 (segment (start 135.768619 89.824149) (end 135.990081 90.045611) (width 0.2032) (layer F.Cu) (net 6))
 (segment (start 135.990081 90.045611) (end 135.990081 106.481521) (width 0.2032) (layer F.Cu) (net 6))
 (segment (start 135.990081 106.481521) (end 135.602618 106.868984) (width 0.2032) (layer F.Cu) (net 6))
 (segment (start 135.602618 106.868984) (end 134.752619 107.718983) (width 0.2032) (layer F.Cu) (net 6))
 (segment (start 133.736619 89.811983) (end 133.736619 97.624133) (width 0.2032) (layer F.Cu) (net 7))
 (segment (start 133.495226 106.436376) (end 133.062618 106.868984) (width 0.2032) (layer F.Cu) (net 7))
 (segment (start 133.736619 97.624133) (end 133.495226 97.865526) (width 0.2032) (layer F.Cu) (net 7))
 (segment (start 133.495226 97.865526) (end 133.495226 106.436376) (width 0.2032) (layer F.Cu) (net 7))
 (segment (start 133.062618 106.868984) (end 132.212619 107.718983) (width 0.2032) (layer F.Cu) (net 7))
 (segment (start 131.704619 89.811983) (end 131.704619 98.897877) (width 0.2032) (layer F.Cu) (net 8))
 (segment (start 131.704619 98.897877) (end 130.82742 99.775076) (width 0.2032) (layer F.Cu) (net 8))
 (segment (start 130.82742 99.775076) (end 130.82742 106.564182) (width 0.2032) (layer F.Cu) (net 8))
 (segment (start 130.82742 106.564182) (end 130.522618 106.868984) (width 0.2032) (layer F.Cu) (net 8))
 (segment (start 130.522618 106.868984) (end 129.672619 107.718983) (width 0.2032) (layer F.Cu) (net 8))
 (segment (start 134.752619 88.033983) (end 134.752619 100.098983) (width 0.2032) (layer F.Cu) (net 9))
 (segment (start 132.720619 88.033983) (end 132.720619 99.590983) (width 0.2032) (layer F.Cu) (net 10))
 (segment (start 132.720619 99.590983) (end 132.212619 100.098983) (width 0.2032) (layer F.Cu) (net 10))
 (segment (start 136.784619 88.033983) (end 136.784619 89.021811) (width 0.2032) (layer F.Cu) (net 11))
 (segment (start 136.784619 89.021811) (end 136.797318 89.03451) (width 0.2032) (layer F.Cu) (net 11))
 (segment (start 136.797318 89.03451) (end 136.797318 97.549845) (width 0.2032) (layer F.Cu) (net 11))
 (segment (start 136.797318 97.549845) (end 137.292619 98.045146) (width 0.2032) (layer F.Cu) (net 11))
 (segment (start 137.292619 98.045146) (end 137.292619 100.098983) (width 0.2032) (layer F.Cu) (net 11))
 (segment (start 130.688619 88.033983) (end 130.688619 99.082983) (width 0.2032) (layer F.Cu) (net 12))
 (segment (start 130.688619 99.082983) (end 129.672619 100.098983) (width 0.2032) (layer F.Cu) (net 12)))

